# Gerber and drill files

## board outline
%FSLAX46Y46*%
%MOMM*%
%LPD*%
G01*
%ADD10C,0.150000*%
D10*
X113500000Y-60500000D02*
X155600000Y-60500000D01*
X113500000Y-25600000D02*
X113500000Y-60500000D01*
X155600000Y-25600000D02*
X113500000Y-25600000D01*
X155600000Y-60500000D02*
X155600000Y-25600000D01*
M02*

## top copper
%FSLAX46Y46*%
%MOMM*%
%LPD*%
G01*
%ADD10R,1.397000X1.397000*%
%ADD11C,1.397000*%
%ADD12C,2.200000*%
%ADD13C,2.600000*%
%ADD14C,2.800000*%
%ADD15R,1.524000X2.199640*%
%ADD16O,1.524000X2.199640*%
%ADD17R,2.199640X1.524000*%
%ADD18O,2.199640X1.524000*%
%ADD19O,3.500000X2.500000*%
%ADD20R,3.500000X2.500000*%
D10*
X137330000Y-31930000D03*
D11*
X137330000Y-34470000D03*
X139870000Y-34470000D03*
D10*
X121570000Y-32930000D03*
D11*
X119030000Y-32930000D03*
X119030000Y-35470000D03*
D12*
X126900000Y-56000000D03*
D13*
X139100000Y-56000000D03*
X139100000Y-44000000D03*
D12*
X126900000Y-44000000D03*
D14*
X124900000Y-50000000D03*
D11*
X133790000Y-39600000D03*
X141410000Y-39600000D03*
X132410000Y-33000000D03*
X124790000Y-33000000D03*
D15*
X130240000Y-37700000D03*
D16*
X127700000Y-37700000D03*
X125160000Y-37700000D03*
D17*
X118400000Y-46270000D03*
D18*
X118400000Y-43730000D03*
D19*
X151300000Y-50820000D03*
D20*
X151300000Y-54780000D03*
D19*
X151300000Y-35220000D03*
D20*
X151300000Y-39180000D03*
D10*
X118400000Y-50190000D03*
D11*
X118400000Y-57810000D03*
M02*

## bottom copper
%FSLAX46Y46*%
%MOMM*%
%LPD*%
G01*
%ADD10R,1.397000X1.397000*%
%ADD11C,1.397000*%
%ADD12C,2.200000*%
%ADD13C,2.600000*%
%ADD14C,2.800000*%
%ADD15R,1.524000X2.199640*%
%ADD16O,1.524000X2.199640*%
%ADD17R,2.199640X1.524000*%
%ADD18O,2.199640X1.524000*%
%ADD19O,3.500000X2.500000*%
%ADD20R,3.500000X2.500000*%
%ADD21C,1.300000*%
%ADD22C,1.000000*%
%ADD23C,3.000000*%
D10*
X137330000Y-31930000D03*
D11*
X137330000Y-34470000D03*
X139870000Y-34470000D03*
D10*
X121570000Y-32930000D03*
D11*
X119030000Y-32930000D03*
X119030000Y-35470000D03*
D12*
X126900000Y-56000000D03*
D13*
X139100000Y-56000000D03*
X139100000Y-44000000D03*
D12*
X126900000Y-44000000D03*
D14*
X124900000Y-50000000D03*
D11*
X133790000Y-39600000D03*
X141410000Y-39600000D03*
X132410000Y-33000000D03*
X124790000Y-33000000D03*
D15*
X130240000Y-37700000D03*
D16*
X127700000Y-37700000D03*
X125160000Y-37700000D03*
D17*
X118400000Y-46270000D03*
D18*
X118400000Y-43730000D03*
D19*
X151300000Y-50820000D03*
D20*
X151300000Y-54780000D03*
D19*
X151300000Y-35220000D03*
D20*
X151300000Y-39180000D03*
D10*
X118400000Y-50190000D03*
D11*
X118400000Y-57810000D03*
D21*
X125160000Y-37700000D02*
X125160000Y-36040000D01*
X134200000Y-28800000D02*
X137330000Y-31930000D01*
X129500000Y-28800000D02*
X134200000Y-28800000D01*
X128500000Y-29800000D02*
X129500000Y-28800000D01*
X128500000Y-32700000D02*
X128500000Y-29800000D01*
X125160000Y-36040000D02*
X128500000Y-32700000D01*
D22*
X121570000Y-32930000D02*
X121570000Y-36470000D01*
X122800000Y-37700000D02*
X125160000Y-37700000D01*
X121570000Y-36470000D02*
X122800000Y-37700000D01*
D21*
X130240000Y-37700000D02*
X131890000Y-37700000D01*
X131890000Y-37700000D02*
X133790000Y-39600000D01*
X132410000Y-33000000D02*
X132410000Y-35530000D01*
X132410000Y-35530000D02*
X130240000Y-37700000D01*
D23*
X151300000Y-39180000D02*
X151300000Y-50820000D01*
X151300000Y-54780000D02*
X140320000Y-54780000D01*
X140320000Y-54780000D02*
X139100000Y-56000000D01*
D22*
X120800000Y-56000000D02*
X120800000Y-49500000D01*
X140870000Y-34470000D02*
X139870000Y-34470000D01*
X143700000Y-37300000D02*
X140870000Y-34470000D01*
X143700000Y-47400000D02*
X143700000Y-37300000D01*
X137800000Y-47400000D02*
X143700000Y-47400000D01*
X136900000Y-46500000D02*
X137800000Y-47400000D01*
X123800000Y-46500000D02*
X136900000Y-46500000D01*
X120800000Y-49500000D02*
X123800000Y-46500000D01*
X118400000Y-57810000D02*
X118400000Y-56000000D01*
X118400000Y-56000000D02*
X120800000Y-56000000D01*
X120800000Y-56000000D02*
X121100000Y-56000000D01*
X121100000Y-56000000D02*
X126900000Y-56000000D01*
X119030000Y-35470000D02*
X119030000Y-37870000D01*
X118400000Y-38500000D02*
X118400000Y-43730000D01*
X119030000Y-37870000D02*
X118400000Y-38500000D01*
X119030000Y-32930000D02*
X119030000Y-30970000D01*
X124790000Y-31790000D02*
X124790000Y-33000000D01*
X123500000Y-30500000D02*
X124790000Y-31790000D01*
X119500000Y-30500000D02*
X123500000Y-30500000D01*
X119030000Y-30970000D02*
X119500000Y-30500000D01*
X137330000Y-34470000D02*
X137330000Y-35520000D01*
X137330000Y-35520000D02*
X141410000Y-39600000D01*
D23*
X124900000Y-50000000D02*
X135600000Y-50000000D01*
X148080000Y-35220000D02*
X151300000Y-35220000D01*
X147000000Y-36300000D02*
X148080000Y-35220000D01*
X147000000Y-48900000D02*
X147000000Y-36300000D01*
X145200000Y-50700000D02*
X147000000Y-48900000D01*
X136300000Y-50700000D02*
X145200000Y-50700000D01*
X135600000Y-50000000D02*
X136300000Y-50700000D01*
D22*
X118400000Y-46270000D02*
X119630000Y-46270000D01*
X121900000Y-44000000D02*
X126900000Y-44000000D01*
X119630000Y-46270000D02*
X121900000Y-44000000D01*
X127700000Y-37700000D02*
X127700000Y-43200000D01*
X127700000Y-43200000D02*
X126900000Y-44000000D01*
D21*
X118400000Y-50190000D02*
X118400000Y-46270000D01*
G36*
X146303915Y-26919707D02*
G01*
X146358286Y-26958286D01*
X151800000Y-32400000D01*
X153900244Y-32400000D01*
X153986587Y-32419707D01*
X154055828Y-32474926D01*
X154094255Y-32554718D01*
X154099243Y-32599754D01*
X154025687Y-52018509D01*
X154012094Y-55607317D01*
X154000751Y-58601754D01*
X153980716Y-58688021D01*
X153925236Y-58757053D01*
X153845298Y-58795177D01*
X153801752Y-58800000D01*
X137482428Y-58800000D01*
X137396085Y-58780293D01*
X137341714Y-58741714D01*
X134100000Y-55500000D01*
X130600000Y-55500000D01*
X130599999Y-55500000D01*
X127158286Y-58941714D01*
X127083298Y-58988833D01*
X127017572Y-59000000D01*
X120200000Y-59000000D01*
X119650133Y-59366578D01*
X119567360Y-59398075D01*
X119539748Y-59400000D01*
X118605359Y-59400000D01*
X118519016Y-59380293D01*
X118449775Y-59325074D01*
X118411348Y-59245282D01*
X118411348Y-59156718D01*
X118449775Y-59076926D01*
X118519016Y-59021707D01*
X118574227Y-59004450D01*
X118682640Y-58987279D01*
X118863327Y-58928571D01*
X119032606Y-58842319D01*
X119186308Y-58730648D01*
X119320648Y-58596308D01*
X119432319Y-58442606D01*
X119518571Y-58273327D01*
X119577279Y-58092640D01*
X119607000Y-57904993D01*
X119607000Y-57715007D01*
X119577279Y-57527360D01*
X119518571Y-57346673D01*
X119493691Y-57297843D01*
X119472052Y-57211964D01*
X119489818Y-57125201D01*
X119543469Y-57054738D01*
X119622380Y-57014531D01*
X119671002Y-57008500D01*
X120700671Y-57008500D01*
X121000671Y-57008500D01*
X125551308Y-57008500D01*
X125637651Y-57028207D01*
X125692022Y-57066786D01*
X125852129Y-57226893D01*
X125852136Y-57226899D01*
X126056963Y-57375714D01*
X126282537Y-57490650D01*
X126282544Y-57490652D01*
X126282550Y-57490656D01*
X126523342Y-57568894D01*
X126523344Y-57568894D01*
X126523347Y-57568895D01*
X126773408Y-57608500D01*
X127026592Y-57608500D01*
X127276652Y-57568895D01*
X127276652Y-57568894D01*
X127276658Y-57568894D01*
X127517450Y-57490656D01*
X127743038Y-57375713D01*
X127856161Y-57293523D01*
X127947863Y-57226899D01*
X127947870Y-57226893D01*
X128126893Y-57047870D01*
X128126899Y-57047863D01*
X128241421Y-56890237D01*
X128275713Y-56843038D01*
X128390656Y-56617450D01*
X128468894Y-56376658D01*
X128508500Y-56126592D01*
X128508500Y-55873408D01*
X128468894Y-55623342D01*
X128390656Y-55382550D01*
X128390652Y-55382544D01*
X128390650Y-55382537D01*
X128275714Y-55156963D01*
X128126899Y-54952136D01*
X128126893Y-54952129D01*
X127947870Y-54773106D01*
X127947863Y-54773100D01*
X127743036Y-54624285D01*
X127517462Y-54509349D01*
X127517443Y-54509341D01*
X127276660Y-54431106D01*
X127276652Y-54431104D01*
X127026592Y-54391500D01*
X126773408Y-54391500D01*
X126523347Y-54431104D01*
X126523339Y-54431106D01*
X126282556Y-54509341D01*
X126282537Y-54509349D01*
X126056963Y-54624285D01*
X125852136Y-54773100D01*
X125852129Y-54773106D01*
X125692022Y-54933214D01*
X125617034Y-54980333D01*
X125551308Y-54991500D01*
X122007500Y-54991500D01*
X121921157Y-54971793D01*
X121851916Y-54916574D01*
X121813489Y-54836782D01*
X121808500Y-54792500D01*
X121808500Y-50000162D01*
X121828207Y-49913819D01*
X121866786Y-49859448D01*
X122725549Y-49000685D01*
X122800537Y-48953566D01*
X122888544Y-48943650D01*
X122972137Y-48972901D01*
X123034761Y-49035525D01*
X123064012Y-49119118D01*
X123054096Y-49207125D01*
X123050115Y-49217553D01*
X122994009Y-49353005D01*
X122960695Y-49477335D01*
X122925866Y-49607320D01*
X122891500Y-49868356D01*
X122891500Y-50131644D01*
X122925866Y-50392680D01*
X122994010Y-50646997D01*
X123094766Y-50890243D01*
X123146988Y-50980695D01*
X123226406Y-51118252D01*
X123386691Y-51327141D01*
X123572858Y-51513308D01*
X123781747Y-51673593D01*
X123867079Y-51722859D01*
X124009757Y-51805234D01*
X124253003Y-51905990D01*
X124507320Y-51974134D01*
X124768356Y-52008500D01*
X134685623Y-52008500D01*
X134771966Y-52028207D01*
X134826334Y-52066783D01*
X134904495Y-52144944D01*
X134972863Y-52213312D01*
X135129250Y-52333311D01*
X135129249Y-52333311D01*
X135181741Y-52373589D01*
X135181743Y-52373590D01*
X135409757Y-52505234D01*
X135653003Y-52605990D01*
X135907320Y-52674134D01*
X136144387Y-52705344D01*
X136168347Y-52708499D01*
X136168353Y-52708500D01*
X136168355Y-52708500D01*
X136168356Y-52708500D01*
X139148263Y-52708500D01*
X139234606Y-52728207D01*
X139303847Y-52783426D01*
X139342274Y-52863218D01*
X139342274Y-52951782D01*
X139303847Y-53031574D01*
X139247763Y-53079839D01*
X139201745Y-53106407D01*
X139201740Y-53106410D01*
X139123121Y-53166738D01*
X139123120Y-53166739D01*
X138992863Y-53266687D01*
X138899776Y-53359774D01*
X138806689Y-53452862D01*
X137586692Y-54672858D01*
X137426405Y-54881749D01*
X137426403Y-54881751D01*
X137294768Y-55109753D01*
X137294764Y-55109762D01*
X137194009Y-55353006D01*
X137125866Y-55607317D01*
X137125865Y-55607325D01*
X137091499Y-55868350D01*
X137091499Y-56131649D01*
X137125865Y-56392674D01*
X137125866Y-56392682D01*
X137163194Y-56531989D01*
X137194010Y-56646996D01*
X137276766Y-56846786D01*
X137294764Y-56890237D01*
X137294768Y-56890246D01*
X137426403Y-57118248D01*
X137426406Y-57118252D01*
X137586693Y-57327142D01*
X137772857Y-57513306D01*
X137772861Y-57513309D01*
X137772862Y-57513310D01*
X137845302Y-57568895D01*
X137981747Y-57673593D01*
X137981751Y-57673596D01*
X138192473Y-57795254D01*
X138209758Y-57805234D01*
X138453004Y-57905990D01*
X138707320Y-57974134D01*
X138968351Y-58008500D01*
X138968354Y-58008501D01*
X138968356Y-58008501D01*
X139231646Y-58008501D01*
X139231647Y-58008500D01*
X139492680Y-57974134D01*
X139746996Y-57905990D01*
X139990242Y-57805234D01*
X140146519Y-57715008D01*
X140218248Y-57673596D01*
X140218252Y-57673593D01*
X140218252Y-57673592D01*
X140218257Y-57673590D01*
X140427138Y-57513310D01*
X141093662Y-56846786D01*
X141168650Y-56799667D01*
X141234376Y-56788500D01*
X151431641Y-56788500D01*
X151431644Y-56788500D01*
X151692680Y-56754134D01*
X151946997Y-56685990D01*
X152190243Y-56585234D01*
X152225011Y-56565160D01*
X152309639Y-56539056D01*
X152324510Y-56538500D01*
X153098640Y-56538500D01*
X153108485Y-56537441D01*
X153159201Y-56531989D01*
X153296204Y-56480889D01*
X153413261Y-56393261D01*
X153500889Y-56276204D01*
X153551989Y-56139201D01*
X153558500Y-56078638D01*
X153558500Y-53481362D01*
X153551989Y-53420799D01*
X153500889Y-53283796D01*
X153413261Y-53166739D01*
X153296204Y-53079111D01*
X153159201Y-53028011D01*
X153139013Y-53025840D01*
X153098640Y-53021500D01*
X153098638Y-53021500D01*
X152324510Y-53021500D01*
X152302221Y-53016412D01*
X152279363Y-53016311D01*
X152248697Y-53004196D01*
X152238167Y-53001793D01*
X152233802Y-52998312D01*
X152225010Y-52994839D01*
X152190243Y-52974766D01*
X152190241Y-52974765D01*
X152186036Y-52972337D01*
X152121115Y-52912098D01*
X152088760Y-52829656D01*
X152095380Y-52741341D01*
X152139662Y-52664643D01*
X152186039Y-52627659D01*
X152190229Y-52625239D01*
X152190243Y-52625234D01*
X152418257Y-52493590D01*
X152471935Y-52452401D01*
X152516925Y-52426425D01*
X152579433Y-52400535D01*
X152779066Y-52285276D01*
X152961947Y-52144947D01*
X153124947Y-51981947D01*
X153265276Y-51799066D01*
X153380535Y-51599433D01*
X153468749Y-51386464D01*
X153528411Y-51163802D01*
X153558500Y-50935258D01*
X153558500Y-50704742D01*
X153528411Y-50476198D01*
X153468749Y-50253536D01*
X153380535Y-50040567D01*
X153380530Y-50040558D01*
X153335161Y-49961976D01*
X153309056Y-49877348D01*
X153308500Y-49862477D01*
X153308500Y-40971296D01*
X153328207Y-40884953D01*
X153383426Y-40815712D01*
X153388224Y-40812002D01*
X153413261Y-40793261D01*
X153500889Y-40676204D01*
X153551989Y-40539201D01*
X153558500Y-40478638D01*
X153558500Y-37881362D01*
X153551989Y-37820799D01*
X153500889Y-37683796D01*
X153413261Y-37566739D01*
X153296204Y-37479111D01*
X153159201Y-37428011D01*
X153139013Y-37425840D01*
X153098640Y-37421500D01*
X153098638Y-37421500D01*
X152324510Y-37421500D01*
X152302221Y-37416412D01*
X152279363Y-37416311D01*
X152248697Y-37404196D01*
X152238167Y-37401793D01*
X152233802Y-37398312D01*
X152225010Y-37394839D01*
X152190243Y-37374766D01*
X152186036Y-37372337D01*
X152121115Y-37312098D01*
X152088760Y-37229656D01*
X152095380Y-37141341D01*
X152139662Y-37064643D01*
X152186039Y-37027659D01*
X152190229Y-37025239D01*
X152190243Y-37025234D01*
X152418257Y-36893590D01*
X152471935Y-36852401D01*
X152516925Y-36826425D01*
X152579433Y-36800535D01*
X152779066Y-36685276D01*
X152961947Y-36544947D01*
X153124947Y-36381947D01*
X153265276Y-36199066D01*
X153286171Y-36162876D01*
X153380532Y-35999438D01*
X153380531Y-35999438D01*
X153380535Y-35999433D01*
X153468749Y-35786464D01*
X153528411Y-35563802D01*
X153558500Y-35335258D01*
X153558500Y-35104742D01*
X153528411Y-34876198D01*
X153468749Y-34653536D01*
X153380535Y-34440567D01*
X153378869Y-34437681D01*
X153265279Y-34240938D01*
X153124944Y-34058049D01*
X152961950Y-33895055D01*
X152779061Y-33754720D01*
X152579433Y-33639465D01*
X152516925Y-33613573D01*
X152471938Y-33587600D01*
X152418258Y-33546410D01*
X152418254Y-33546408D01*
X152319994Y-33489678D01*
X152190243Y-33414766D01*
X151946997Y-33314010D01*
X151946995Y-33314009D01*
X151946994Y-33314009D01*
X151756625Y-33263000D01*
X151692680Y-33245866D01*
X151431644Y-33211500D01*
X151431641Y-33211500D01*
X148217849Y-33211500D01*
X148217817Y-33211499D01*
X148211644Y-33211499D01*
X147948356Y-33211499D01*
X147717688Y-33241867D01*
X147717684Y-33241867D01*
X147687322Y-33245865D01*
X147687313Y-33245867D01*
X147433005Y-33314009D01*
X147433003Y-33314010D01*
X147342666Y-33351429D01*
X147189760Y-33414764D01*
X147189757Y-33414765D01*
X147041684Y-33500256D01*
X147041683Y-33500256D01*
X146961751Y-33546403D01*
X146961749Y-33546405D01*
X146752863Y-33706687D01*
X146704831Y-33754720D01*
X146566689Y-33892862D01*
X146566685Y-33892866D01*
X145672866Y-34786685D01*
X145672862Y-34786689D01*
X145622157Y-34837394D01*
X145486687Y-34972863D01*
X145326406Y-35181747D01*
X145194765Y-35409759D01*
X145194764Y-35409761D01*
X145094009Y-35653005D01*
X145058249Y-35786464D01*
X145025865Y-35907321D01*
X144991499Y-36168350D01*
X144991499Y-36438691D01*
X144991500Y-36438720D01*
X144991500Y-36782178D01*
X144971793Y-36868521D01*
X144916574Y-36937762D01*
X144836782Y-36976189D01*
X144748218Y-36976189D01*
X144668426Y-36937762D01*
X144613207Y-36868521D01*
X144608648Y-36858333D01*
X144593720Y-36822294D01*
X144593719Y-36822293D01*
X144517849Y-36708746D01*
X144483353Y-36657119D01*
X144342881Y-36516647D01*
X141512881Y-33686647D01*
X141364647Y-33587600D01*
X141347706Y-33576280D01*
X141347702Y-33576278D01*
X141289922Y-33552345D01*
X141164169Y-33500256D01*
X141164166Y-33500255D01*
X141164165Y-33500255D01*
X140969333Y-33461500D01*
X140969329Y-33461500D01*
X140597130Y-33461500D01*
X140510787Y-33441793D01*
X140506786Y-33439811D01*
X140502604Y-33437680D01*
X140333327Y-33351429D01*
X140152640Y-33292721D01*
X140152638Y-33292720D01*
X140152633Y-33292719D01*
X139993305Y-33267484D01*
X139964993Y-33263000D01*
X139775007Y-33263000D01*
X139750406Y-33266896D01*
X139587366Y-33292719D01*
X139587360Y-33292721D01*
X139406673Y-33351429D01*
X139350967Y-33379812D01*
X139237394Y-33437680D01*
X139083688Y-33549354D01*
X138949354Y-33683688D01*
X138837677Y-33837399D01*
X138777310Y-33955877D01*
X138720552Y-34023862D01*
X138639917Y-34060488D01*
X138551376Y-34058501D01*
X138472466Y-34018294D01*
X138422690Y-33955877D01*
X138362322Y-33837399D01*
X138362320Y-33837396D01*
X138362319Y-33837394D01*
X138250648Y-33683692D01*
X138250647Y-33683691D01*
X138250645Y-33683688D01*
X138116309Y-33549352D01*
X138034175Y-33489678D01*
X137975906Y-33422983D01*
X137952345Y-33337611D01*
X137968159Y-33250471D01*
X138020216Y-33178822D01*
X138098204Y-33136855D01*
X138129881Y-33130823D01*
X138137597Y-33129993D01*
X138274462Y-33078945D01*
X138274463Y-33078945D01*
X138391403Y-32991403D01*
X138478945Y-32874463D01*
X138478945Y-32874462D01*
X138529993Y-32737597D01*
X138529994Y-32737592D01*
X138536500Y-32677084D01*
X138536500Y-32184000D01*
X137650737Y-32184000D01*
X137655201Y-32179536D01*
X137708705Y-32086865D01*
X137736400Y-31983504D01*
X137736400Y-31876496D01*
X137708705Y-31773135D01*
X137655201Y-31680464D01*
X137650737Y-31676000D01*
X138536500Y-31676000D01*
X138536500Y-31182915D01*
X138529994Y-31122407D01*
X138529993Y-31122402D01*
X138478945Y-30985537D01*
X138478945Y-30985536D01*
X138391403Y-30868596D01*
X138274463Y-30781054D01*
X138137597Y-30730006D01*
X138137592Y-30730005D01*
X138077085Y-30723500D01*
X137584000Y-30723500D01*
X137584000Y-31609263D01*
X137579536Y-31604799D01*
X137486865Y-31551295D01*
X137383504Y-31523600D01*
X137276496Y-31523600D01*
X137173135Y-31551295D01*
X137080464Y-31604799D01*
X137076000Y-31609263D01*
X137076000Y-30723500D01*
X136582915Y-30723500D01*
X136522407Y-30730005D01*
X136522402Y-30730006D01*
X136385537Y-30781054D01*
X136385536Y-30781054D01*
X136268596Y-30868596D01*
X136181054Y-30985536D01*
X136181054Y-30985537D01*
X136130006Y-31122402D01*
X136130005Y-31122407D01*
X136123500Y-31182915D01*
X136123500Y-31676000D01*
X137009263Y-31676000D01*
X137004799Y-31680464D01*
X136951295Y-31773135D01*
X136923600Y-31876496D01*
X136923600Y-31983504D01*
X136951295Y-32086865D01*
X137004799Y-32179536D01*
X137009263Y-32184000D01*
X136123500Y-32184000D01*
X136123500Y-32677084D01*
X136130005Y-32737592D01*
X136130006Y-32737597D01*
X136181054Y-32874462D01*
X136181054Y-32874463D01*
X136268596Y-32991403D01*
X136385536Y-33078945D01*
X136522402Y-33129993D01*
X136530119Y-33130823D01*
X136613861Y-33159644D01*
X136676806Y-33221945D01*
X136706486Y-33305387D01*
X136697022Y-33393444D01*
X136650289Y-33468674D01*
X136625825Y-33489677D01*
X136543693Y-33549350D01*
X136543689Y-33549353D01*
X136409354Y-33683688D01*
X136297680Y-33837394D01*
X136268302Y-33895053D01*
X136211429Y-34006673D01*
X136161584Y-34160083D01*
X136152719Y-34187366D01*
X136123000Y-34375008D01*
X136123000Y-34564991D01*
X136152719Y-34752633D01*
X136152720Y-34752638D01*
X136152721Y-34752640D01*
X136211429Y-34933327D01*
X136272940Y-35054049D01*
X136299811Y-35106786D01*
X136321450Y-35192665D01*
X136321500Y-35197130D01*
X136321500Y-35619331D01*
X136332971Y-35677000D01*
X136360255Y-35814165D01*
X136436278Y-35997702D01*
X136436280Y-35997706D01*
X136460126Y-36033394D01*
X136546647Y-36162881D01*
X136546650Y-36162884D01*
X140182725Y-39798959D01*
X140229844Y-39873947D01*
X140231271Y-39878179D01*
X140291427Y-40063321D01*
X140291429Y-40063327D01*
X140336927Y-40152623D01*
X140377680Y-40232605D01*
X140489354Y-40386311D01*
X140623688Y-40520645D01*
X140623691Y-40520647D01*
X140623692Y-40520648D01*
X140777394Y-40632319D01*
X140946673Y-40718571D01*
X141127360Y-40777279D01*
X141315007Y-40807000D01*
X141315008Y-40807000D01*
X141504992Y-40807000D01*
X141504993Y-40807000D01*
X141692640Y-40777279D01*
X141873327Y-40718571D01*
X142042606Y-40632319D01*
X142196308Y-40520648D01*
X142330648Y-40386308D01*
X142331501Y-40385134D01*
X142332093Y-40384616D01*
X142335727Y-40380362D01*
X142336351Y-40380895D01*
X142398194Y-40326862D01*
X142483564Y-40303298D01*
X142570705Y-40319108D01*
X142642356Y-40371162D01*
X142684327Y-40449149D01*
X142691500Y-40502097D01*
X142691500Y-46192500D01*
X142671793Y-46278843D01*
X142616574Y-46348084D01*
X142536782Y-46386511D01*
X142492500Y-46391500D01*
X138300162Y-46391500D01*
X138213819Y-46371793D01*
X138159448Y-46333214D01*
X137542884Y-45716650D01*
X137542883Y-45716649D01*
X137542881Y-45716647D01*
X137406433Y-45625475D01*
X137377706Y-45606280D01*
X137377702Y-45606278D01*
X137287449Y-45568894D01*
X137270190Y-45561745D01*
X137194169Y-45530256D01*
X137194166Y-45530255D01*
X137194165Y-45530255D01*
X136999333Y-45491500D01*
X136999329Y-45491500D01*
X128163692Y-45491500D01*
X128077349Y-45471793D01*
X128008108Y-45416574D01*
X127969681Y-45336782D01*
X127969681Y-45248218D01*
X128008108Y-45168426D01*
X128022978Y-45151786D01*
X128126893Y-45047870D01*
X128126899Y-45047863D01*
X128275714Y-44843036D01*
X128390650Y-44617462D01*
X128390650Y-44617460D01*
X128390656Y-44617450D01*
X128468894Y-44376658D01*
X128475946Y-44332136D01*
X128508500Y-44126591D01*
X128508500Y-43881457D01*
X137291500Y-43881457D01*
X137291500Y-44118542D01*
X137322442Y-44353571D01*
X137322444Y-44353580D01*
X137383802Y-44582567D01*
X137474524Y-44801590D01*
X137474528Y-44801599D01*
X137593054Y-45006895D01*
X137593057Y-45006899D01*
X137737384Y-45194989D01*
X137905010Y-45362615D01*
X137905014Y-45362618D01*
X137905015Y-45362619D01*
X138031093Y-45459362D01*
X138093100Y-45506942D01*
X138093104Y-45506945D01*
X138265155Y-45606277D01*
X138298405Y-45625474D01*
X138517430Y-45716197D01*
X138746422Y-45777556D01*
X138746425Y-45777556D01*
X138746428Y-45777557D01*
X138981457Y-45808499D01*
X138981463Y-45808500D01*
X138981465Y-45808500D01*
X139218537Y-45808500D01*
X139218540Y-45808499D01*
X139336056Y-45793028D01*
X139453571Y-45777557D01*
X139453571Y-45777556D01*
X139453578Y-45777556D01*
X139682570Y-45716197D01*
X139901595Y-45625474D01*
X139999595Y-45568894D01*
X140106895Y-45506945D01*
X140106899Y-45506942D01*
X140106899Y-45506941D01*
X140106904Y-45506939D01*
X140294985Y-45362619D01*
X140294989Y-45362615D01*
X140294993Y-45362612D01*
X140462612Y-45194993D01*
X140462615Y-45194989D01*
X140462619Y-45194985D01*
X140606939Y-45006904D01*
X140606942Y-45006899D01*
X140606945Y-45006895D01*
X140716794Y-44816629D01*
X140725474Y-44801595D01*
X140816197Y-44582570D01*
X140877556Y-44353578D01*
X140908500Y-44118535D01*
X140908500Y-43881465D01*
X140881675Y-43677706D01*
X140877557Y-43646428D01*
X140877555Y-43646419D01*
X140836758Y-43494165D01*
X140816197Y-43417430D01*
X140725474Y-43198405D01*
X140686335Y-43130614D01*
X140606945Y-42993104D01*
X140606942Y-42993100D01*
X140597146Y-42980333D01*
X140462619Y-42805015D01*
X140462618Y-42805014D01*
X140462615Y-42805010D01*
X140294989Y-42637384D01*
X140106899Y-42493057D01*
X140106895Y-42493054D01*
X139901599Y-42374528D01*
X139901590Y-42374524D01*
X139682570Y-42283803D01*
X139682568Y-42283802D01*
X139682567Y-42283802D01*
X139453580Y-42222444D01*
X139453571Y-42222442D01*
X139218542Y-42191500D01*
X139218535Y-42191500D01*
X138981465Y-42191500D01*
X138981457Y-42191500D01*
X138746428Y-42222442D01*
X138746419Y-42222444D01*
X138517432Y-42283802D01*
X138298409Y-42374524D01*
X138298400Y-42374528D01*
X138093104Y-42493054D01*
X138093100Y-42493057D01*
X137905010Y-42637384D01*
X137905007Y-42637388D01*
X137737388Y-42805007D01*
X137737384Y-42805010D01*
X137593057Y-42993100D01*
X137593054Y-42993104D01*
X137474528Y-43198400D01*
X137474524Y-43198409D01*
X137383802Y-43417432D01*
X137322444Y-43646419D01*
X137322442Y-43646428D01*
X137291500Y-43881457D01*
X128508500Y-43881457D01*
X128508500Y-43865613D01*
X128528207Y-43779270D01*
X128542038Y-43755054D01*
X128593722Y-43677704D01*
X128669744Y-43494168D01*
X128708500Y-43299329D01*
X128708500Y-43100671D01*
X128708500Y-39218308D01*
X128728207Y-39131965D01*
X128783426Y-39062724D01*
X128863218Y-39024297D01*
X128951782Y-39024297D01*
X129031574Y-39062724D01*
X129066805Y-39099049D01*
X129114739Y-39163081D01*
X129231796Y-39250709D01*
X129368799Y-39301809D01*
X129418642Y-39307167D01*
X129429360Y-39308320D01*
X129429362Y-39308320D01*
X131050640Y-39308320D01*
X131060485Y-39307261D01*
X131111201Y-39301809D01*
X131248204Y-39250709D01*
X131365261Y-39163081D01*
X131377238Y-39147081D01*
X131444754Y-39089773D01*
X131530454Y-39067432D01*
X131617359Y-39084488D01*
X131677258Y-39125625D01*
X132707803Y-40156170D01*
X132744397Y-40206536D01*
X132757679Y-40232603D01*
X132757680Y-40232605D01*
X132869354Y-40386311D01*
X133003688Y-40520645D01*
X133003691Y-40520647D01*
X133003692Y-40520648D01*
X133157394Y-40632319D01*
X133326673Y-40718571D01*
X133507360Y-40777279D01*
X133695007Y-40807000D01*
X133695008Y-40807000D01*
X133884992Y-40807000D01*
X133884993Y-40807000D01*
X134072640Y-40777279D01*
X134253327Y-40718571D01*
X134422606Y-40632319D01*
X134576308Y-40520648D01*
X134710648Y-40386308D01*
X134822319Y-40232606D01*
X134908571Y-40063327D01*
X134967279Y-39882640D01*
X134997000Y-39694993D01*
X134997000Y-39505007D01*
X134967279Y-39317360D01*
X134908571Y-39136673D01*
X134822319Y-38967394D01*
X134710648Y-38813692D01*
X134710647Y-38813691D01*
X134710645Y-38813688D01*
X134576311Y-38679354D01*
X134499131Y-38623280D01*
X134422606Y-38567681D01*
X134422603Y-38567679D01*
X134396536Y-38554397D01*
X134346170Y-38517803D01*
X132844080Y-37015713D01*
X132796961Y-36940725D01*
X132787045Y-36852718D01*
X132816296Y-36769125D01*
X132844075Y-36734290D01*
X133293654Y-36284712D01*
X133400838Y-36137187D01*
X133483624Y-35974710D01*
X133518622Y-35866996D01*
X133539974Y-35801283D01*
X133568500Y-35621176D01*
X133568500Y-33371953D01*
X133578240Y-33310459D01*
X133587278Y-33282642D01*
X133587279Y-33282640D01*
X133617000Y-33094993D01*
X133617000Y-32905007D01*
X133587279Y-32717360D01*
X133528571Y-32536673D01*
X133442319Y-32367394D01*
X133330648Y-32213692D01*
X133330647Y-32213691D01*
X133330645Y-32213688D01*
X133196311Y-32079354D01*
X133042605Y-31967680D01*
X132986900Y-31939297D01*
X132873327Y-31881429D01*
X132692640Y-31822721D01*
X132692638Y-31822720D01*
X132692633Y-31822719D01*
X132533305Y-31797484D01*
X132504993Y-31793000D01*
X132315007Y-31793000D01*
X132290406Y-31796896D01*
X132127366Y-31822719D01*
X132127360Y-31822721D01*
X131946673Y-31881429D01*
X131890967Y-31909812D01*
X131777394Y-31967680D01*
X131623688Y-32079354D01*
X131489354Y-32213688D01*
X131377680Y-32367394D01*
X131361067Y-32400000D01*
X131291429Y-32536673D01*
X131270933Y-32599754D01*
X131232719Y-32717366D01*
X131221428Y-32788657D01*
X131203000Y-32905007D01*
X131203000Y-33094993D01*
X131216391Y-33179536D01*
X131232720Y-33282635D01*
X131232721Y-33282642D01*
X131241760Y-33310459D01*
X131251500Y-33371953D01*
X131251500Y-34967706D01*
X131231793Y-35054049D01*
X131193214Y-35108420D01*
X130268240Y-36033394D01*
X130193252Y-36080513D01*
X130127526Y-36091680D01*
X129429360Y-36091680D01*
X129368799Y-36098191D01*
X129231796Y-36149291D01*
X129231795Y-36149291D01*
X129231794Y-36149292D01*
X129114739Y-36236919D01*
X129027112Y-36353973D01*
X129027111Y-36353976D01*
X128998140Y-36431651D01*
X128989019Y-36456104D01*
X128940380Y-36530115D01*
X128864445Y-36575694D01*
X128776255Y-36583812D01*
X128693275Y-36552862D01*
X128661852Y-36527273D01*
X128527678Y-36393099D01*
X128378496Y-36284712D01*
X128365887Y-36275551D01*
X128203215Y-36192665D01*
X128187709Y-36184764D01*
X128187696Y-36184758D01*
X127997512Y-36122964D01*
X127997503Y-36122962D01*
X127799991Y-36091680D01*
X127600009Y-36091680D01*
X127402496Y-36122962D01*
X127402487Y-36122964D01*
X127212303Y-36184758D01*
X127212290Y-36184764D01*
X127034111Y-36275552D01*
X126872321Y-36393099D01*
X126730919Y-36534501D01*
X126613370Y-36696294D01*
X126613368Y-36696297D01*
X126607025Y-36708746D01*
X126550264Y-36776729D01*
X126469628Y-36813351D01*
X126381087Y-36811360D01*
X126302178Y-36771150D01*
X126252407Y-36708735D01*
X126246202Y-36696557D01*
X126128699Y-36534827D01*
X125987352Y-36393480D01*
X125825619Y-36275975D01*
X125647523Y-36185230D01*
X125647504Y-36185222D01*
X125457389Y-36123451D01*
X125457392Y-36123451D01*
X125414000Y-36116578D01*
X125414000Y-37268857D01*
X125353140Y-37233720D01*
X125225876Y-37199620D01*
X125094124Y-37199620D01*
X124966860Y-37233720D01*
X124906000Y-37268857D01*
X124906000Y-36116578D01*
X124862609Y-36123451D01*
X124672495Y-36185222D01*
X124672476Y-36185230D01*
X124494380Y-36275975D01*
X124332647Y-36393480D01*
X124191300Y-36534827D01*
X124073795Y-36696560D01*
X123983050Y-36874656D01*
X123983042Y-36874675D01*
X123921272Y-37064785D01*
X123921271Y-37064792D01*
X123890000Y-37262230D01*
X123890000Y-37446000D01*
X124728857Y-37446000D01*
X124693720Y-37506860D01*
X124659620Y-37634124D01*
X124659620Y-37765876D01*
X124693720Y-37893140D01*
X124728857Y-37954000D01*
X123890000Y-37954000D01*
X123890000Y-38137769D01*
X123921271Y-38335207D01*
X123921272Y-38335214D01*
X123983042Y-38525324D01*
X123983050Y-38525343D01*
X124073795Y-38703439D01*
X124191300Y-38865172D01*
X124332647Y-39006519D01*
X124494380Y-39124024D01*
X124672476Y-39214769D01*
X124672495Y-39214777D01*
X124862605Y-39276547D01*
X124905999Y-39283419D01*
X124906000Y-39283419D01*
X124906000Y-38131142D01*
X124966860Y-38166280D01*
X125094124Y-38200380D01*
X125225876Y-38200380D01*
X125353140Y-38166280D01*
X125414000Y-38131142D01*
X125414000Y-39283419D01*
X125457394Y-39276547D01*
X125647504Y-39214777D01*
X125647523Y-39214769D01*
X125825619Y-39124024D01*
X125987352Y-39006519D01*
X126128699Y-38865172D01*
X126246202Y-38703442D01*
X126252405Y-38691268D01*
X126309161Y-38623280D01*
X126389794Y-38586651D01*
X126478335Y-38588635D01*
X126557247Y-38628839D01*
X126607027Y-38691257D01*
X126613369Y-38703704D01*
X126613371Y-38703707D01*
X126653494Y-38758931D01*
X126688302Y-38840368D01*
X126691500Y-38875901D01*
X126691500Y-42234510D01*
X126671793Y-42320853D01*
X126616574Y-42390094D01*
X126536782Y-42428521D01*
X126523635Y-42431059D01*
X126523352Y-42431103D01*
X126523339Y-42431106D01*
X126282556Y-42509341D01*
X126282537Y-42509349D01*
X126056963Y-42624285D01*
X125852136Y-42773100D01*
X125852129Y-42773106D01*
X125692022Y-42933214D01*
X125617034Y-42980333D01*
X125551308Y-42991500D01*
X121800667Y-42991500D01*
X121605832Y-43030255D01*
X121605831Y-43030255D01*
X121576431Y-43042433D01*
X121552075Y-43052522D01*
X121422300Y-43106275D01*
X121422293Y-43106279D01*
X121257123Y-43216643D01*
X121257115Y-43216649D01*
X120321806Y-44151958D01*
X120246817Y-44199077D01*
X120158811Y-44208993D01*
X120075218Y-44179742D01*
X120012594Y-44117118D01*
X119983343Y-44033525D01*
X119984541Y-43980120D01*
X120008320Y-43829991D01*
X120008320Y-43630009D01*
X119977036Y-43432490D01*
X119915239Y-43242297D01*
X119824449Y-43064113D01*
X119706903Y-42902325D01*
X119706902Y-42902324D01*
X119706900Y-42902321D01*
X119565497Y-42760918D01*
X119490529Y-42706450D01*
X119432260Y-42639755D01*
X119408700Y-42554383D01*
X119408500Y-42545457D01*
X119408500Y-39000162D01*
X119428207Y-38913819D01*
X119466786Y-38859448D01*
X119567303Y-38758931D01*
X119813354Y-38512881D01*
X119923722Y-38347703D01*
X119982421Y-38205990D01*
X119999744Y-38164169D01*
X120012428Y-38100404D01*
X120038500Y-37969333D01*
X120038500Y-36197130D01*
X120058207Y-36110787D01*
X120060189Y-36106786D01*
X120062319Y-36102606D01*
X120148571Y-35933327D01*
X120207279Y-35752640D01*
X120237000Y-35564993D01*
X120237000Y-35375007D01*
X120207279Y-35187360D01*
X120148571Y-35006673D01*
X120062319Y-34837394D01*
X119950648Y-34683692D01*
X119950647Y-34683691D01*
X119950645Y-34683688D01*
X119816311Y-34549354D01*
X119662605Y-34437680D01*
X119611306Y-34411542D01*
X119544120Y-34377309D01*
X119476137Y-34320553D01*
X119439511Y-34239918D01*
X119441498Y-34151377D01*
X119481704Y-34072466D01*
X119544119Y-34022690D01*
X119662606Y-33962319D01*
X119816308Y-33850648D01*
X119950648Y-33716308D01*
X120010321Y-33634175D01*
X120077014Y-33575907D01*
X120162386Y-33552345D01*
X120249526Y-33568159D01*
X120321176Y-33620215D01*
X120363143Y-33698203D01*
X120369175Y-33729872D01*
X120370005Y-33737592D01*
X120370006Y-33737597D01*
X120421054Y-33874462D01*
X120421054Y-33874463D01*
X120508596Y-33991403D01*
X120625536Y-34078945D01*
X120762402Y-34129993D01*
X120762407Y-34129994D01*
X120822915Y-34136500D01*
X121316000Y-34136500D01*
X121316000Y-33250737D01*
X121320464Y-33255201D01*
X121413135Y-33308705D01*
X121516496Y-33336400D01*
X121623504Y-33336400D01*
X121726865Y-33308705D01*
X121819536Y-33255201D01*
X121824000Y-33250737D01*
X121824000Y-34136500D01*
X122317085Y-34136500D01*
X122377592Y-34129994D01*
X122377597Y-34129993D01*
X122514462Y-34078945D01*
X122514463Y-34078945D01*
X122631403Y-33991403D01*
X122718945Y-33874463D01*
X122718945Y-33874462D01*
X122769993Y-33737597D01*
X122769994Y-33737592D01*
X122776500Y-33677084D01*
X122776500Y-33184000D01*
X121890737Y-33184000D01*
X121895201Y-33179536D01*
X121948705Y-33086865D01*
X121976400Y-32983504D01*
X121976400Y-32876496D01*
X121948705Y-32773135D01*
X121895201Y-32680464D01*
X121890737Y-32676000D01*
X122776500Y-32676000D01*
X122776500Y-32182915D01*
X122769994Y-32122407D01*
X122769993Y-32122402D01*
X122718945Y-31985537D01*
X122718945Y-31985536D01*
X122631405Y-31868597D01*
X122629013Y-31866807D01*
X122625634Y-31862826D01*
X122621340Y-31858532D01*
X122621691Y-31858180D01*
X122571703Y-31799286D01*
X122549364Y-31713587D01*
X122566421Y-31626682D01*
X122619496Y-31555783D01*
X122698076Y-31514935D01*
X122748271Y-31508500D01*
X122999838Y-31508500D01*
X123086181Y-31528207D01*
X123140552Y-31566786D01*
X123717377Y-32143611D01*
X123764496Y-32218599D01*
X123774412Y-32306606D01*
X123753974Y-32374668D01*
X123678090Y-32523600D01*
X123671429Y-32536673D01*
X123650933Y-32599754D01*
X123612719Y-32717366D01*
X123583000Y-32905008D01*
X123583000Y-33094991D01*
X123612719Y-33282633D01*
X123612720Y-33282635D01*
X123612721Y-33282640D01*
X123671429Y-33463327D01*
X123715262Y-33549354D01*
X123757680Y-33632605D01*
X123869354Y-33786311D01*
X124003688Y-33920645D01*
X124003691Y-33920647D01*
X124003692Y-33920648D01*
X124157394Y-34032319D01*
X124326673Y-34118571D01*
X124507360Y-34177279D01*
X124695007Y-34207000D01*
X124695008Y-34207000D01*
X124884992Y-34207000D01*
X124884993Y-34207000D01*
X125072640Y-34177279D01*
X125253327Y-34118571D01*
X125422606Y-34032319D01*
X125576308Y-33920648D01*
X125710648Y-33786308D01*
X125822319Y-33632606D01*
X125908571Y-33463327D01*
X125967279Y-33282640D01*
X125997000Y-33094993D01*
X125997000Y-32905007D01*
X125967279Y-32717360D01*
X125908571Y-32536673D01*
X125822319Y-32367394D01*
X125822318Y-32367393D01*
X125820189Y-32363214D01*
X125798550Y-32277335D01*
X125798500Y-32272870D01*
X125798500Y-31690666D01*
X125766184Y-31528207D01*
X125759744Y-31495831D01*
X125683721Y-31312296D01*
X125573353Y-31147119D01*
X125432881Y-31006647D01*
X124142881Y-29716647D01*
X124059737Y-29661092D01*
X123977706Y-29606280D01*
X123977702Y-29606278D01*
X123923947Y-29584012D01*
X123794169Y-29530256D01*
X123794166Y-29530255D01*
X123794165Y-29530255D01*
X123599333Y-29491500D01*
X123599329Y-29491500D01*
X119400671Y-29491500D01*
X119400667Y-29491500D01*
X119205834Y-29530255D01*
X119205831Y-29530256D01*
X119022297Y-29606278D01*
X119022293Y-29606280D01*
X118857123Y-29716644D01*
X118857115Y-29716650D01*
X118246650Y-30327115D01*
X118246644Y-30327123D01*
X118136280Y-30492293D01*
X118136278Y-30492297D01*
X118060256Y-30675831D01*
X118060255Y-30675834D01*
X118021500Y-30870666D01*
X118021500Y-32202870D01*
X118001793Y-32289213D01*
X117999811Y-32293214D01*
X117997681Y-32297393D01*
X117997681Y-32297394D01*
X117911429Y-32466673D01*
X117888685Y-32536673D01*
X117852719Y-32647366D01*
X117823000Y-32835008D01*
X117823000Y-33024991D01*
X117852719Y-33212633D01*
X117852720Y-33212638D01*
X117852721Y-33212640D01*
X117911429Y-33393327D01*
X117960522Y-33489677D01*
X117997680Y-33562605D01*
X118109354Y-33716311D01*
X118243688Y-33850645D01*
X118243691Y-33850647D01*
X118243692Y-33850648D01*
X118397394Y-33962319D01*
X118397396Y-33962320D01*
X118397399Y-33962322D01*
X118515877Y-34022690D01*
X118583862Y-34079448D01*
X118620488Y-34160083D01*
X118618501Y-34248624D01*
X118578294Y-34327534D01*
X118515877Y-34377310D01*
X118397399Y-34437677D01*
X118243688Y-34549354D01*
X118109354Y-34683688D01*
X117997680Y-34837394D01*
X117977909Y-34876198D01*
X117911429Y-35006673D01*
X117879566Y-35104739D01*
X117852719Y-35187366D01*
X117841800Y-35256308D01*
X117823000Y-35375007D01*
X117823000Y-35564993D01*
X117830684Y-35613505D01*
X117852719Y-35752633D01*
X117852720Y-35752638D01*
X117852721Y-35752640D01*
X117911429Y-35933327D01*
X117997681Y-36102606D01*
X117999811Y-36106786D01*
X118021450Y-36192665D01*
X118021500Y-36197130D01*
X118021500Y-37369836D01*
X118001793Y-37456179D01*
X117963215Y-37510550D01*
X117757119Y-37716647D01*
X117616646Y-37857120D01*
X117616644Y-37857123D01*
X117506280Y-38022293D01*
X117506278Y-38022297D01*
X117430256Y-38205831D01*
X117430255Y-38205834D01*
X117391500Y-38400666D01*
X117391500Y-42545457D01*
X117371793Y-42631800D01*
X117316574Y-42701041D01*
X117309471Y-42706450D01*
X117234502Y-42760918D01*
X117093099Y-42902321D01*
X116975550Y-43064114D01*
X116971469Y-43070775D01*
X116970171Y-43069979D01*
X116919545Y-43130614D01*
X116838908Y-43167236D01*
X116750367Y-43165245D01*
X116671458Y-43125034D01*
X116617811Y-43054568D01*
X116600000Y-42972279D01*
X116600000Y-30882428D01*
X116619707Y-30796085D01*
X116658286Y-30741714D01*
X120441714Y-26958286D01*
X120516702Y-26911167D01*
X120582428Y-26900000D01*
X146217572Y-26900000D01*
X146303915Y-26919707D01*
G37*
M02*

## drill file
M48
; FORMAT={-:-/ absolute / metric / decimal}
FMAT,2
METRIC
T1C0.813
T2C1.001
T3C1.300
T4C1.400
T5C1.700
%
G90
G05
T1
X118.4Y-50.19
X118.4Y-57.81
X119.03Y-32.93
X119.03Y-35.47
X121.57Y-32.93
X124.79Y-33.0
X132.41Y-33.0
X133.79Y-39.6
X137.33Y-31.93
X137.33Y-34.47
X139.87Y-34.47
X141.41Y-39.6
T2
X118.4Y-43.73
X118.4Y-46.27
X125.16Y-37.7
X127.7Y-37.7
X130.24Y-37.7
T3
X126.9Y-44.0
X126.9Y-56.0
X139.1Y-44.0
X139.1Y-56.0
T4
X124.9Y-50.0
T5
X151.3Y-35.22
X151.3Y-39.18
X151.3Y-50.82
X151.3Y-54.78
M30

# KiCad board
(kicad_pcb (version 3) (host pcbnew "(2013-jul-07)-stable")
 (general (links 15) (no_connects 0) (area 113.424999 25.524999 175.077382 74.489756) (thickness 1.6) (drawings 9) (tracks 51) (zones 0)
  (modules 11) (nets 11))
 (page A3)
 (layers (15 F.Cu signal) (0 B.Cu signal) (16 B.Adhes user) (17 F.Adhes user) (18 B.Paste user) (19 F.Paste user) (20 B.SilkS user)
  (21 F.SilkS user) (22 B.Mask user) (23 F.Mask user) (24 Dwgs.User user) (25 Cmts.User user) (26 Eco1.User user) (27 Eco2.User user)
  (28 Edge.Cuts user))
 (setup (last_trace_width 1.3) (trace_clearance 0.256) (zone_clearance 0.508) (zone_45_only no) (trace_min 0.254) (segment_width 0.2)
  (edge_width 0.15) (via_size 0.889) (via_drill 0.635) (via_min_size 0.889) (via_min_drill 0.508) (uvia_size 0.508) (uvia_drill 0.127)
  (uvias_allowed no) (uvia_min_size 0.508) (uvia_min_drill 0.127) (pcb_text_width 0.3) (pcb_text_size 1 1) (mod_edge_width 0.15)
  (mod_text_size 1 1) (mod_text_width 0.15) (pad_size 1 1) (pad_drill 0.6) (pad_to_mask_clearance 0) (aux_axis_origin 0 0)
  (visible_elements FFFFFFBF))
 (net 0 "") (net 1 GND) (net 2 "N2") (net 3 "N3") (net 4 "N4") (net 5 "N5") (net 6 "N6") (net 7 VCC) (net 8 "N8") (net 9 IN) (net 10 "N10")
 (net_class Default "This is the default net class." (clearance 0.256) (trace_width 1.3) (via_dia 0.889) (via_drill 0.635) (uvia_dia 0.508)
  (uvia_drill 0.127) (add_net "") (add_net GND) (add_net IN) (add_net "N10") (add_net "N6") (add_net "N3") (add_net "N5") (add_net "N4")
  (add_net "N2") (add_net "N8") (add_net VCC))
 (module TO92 (layer F.Cu) (at 138.6 33.2 90)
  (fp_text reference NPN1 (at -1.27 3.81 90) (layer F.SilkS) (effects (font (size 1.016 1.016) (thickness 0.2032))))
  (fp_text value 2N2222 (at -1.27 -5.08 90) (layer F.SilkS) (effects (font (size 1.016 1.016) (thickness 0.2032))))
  (pad 1 thru_hole rect (at 1.27 -1.27 90) (size 1.397 1.397) (drill 0.8128) (layers *.Cu *.Mask F.SilkS) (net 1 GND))
  (pad 2 thru_hole circle (at -1.27 -1.27 90) (size 1.397 1.397) (drill 0.8128) (layers *.Cu *.Mask F.SilkS) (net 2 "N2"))
  (pad 3 thru_hole circle (at -1.27 1.27 90) (size 1.397 1.397) (drill 0.8128) (layers *.Cu *.Mask F.SilkS) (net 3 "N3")))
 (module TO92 (layer F.Cu) (at 120.3 34.2)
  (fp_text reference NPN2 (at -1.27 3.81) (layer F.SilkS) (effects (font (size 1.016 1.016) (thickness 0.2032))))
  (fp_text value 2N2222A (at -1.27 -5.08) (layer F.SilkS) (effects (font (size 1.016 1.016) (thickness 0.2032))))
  (pad 1 thru_hole rect (at 1.27 -1.27) (size 1.397 1.397) (drill 0.8128) (layers *.Cu *.Mask F.SilkS) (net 1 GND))
  (pad 2 thru_hole circle (at -1.27 -1.27) (size 1.397 1.397) (drill 0.8128) (layers *.Cu *.Mask F.SilkS) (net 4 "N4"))
  (pad 3 thru_hole circle (at -1.27 1.27) (size 1.397 1.397) (drill 0.8128) (layers *.Cu *.Mask F.SilkS) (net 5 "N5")))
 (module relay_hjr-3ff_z (layer F.Cu) (at 133 50 90)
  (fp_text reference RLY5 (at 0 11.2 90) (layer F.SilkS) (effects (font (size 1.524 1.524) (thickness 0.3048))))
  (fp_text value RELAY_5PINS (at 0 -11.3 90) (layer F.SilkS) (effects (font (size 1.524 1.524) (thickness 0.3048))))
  (pad 2 thru_hole circle (at -6 -6.1 90) (size 2.2 2.2) (drill 1.3) (layers *.Cu) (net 3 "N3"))
  (pad 3 thru_hole circle (at -6 6.1 90) (size 2.6 2.6) (drill 1.3) (layers *.Cu) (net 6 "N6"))
  (pad 4 thru_hole circle (at 6 6.1 90) (size 2.6 2.6) (drill 1.3) (layers *.Cu))
  (pad 5 thru_hole circle (at 6 -6.1 90) (size 2.2 2.2) (drill 1.3) (layers *.Cu) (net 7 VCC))
  (pad 1 thru_hole circle (at 0 -8.1 90) (size 2.8 2.8) (drill 1.4) (layers *.Cu) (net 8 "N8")))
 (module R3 (layer F.Cu) (at 137.6 39.6) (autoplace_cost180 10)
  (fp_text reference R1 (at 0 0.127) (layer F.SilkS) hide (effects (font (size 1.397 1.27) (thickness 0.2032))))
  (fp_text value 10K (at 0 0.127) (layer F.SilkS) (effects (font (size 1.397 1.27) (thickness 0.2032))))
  (pad 1 thru_hole circle (at -3.81 0) (size 1.397 1.397) (drill 0.8128) (layers *.Cu *.Mask F.SilkS) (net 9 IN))
  (pad 2 thru_hole circle (at 3.81 0) (size 1.397 1.397) (drill 0.8128) (layers *.Cu *.Mask F.SilkS) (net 2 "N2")))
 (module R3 (layer F.Cu) (at 128.6 33 180) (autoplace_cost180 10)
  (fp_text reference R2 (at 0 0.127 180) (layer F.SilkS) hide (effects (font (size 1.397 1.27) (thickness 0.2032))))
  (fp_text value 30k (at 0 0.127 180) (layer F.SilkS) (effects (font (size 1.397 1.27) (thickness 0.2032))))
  (pad 1 thru_hole circle (at -3.81 0 180) (size 1.397 1.397) (drill 0.8128) (layers *.Cu *.Mask F.SilkS) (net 9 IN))
  (pad 2 thru_hole circle (at 3.81 0 180) (size 1.397 1.397) (drill 0.8128) (layers *.Cu *.Mask F.SilkS) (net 4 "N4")))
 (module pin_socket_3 (layer F.Cu) (at 127.7 37.7 180)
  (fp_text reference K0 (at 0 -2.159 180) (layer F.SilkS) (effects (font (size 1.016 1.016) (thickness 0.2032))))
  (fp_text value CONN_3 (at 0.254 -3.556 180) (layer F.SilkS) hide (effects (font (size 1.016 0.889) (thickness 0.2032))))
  (pad 1 thru_hole rect (at -2.54 0 180) (size 1.524 2.19964) (drill 1.00076) (layers *.Cu *.Mask F.SilkS) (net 9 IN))
  (pad 2 thru_hole oval (at 0 0 180) (size 1.524 2.19964) (drill 1.00076) (layers *.Cu *.Mask F.SilkS) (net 7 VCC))
  (pad 3 thru_hole oval (at 2.54 0 180) (size 1.524 2.19964) (drill 1.00076) (layers *.Cu *.Mask F.SilkS) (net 1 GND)))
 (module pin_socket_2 (layer F.Cu) (at 118.4 45 90)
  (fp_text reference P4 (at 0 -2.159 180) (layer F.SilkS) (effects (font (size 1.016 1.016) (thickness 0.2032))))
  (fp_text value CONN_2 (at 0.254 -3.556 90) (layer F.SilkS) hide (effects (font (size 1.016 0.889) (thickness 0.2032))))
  (pad 1 thru_hole rect (at -1.27 0 90) (size 1.524 2.19964) (drill 1.00076) (layers *.Cu *.Mask F.SilkS) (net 7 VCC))
  (pad 2 thru_hole oval (at 1.27 0 90) (size 1.524 2.19964) (drill 1.00076) (layers *.Cu *.Mask F.SilkS) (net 5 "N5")))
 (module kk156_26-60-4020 (layer F.Cu) (at 151.3 52.8 270)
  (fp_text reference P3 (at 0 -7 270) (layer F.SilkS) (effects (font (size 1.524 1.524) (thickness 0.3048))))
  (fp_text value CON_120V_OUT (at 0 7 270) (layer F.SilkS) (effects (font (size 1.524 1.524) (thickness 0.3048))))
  (pad 2 thru_hole oval (at -1.98 0 270) (size 2.5 3.5) (drill 1.7) (layers *.Cu *.Mask F.SilkS) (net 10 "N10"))
  (pad 1 thru_hole rect (at 1.98 0 270) (size 2.5 3.5) (drill 1.7) (layers *.Cu *.Mask F.SilkS) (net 6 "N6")))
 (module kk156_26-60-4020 (layer F.Cu) (at 151.3 37.2 270)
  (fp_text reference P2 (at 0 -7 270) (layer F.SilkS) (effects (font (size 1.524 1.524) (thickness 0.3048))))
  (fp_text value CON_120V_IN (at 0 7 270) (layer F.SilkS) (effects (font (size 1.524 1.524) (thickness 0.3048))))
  (pad 2 thru_hole oval (at -1.98 0 270) (size 2.5 3.5) (drill 1.7) (layers *.Cu *.Mask F.SilkS) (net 8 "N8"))
  (pad 1 thru_hole rect (at 1.98 0 270) (size 2.5 3.5) (drill 1.7) (layers *.Cu *.Mask F.SilkS) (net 10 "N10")))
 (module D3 (layer F.Cu) (at 118.4 54 90)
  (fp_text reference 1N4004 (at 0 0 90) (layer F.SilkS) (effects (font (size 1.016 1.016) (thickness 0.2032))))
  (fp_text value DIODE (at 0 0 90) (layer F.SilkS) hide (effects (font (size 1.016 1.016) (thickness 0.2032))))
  (pad 2 thru_hole rect (at 3.81 0 90) (size 1.397 1.397) (drill 0.8128) (layers *.Cu *.Mask F.SilkS) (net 7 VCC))
  (pad 1 thru_hole circle (at -3.81 0 90) (size 1.397 1.397) (drill 0.8128) (layers *.Cu *.Mask F.SilkS) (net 3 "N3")))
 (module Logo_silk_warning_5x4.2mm (layer F.Cu) (at 142.9 30.3 90)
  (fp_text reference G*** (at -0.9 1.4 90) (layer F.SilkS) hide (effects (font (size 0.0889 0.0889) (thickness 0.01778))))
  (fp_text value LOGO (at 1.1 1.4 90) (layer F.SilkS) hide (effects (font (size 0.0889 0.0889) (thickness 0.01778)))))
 (gr_line (start 113.5 60.5) (end 155.6 60.5) (angle 90) (layer Edge.Cuts) (width 0.15))
 (gr_line (start 113.5 25.6) (end 113.5 60.5) (angle 90) (layer Edge.Cuts) (width 0.15))
 (gr_line (start 155.6 25.6) (end 113.5 25.6) (angle 90) (layer Edge.Cuts) (width 0.15))
 (gr_line (start 155.6 60.5) (end 155.6 25.6) (angle 90) (layer Edge.Cuts) (width 0.15))
 (segment (start 125.16 37.7) (end 125.16 36.04) (width 1.3) (layer B.Cu) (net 1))
 (segment (start 134.2 28.8) (end 137.33 31.93) (width 1.3) (layer B.Cu) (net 1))
 (segment (start 129.5 28.8) (end 134.2 28.8) (width 1.3) (layer B.Cu) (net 1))
 (segment (start 128.5 29.8) (end 129.5 28.8) (width 1.3) (layer B.Cu) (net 1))
 (segment (start 128.5 32.7) (end 128.5 29.8) (width 1.3) (layer B.Cu) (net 1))
 (segment (start 125.16 36.04) (end 128.5 32.7) (width 1.3) (layer B.Cu) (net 1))
 (segment (start 121.57 32.93) (end 121.57 36.47) (width 1) (layer B.Cu) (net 1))
 (segment (start 122.8 37.7) (end 125.16 37.7) (width 1) (layer B.Cu) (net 1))
 (segment (start 121.57 36.47) (end 122.8 37.7) (width 1) (layer B.Cu) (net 1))
 (segment (start 130.24 37.7) (end 131.89 37.7) (width 1.3) (layer B.Cu) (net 9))
 (segment (start 131.89 37.7) (end 133.79 39.6) (width 1.3) (layer B.Cu) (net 9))
 (segment (start 132.41 33) (end 132.41 35.53) (width 1.3) (layer B.Cu) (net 9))
 (segment (start 132.41 35.53) (end 130.24 37.7) (width 1.3) (layer B.Cu) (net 9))
 (segment (start 151.3 39.18) (end 151.3 50.82) (width 3) (layer B.Cu) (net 10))
 (segment (start 151.3 54.78) (end 140.32 54.78) (width 3) (layer B.Cu) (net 6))
 (segment (start 140.32 54.78) (end 139.1 56) (width 3) (layer B.Cu) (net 6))
 (segment (start 120.8 56) (end 120.8 49.5) (width 1) (layer B.Cu) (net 3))
 (segment (start 140.87 34.47) (end 139.87 34.47) (width 1) (layer B.Cu) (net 3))
 (segment (start 143.7 37.3) (end 140.87 34.47) (width 1) (layer B.Cu) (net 3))
 (segment (start 143.7 47.4) (end 143.7 37.3) (width 1) (layer B.Cu) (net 3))
 (segment (start 137.8 47.4) (end 143.7 47.4) (width 1) (layer B.Cu) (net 3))
 (segment (start 136.9 46.5) (end 137.8 47.4) (width 1) (layer B.Cu) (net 3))
 (segment (start 123.8 46.5) (end 136.9 46.5) (width 1) (layer B.Cu) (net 3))
 (segment (start 120.8 49.5) (end 123.8 46.5) (width 1) (layer B.Cu) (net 3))
 (segment (start 118.4 57.81) (end 118.4 56) (width 1) (layer B.Cu) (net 3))
 (segment (start 118.4 56) (end 120.8 56) (width 1) (layer B.Cu) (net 3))
 (segment (start 120.8 56) (end 121.1 56) (width 1) (layer B.Cu) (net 3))
 (segment (start 121.1 56) (end 126.9 56) (width 1) (layer B.Cu) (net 3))
 (segment (start 119.03 35.47) (end 119.03 37.87) (width 1) (layer B.Cu) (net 5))
 (segment (start 118.4 38.5) (end 118.4 43.73) (width 1) (layer B.Cu) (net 5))
 (segment (start 119.03 37.87) (end 118.4 38.5) (width 1) (layer B.Cu) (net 5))
 (segment (start 119.03 32.93) (end 119.03 30.97) (width 1) (layer B.Cu) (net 4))
 (segment (start 124.79 31.79) (end 124.79 33) (width 1) (layer B.Cu) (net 4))
 (segment (start 123.5 30.5) (end 124.79 31.79) (width 1) (layer B.Cu) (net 4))
 (segment (start 119.5 30.5) (end 123.5 30.5) (width 1) (layer B.Cu) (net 4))
 (segment (start 119.03 30.97) (end 119.5 30.5) (width 1) (layer B.Cu) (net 4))
 (segment (start 137.33 34.47) (end 137.33 35.52) (width 1) (layer B.Cu) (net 2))
 (segment (start 137.33 35.52) (end 141.41 39.6) (width 1) (layer B.Cu) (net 2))
 (segment (start 124.9 50) (end 135.6 50) (width 3) (layer B.Cu) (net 8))
 (segment (start 148.08 35.22) (end 151.3 35.22) (width 3) (layer B.Cu) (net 8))
 (segment (start 147 36.3) (end 148.08 35.22) (width 3) (layer B.Cu) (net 8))
 (segment (start 147 48.9) (end 147 36.3) (width 3) (layer B.Cu) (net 8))
 (segment (start 145.2 50.7) (end 147 48.9) (width 3) (layer B.Cu) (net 8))
 (segment (start 136.3 50.7) (end 145.2 50.7) (width 3) (layer B.Cu) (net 8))
 (segment (start 135.6 50) (end 136.3 50.7) (width 3) (layer B.Cu) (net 8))
 (segment (start 118.4 46.27) (end 119.63 46.27) (width 1) (layer B.Cu) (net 7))
 (segment (start 121.9 44) (end 126.9 44) (width 1) (layer B.Cu) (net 7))
 (segment (start 119.63 46.27) (end 121.9 44) (width 1) (layer B.Cu) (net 7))
 (segment (start 127.7 37.7) (end 127.7 43.2) (width 1) (layer B.Cu) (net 7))
 (segment (start 127.7 43.2) (end 126.9 44) (width 1) (layer B.Cu) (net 7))
 (segment (start 118.4 50.19) (end 118.4 46.27) (width 1.3) (layer B.Cu) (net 7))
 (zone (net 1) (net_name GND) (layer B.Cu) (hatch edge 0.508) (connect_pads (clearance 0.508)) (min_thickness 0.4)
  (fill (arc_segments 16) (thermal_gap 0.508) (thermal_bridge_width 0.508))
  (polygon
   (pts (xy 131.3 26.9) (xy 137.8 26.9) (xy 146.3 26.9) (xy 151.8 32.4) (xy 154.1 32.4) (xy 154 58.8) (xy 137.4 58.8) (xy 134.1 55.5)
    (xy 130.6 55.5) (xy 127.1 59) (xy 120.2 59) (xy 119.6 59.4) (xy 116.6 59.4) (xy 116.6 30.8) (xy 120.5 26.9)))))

